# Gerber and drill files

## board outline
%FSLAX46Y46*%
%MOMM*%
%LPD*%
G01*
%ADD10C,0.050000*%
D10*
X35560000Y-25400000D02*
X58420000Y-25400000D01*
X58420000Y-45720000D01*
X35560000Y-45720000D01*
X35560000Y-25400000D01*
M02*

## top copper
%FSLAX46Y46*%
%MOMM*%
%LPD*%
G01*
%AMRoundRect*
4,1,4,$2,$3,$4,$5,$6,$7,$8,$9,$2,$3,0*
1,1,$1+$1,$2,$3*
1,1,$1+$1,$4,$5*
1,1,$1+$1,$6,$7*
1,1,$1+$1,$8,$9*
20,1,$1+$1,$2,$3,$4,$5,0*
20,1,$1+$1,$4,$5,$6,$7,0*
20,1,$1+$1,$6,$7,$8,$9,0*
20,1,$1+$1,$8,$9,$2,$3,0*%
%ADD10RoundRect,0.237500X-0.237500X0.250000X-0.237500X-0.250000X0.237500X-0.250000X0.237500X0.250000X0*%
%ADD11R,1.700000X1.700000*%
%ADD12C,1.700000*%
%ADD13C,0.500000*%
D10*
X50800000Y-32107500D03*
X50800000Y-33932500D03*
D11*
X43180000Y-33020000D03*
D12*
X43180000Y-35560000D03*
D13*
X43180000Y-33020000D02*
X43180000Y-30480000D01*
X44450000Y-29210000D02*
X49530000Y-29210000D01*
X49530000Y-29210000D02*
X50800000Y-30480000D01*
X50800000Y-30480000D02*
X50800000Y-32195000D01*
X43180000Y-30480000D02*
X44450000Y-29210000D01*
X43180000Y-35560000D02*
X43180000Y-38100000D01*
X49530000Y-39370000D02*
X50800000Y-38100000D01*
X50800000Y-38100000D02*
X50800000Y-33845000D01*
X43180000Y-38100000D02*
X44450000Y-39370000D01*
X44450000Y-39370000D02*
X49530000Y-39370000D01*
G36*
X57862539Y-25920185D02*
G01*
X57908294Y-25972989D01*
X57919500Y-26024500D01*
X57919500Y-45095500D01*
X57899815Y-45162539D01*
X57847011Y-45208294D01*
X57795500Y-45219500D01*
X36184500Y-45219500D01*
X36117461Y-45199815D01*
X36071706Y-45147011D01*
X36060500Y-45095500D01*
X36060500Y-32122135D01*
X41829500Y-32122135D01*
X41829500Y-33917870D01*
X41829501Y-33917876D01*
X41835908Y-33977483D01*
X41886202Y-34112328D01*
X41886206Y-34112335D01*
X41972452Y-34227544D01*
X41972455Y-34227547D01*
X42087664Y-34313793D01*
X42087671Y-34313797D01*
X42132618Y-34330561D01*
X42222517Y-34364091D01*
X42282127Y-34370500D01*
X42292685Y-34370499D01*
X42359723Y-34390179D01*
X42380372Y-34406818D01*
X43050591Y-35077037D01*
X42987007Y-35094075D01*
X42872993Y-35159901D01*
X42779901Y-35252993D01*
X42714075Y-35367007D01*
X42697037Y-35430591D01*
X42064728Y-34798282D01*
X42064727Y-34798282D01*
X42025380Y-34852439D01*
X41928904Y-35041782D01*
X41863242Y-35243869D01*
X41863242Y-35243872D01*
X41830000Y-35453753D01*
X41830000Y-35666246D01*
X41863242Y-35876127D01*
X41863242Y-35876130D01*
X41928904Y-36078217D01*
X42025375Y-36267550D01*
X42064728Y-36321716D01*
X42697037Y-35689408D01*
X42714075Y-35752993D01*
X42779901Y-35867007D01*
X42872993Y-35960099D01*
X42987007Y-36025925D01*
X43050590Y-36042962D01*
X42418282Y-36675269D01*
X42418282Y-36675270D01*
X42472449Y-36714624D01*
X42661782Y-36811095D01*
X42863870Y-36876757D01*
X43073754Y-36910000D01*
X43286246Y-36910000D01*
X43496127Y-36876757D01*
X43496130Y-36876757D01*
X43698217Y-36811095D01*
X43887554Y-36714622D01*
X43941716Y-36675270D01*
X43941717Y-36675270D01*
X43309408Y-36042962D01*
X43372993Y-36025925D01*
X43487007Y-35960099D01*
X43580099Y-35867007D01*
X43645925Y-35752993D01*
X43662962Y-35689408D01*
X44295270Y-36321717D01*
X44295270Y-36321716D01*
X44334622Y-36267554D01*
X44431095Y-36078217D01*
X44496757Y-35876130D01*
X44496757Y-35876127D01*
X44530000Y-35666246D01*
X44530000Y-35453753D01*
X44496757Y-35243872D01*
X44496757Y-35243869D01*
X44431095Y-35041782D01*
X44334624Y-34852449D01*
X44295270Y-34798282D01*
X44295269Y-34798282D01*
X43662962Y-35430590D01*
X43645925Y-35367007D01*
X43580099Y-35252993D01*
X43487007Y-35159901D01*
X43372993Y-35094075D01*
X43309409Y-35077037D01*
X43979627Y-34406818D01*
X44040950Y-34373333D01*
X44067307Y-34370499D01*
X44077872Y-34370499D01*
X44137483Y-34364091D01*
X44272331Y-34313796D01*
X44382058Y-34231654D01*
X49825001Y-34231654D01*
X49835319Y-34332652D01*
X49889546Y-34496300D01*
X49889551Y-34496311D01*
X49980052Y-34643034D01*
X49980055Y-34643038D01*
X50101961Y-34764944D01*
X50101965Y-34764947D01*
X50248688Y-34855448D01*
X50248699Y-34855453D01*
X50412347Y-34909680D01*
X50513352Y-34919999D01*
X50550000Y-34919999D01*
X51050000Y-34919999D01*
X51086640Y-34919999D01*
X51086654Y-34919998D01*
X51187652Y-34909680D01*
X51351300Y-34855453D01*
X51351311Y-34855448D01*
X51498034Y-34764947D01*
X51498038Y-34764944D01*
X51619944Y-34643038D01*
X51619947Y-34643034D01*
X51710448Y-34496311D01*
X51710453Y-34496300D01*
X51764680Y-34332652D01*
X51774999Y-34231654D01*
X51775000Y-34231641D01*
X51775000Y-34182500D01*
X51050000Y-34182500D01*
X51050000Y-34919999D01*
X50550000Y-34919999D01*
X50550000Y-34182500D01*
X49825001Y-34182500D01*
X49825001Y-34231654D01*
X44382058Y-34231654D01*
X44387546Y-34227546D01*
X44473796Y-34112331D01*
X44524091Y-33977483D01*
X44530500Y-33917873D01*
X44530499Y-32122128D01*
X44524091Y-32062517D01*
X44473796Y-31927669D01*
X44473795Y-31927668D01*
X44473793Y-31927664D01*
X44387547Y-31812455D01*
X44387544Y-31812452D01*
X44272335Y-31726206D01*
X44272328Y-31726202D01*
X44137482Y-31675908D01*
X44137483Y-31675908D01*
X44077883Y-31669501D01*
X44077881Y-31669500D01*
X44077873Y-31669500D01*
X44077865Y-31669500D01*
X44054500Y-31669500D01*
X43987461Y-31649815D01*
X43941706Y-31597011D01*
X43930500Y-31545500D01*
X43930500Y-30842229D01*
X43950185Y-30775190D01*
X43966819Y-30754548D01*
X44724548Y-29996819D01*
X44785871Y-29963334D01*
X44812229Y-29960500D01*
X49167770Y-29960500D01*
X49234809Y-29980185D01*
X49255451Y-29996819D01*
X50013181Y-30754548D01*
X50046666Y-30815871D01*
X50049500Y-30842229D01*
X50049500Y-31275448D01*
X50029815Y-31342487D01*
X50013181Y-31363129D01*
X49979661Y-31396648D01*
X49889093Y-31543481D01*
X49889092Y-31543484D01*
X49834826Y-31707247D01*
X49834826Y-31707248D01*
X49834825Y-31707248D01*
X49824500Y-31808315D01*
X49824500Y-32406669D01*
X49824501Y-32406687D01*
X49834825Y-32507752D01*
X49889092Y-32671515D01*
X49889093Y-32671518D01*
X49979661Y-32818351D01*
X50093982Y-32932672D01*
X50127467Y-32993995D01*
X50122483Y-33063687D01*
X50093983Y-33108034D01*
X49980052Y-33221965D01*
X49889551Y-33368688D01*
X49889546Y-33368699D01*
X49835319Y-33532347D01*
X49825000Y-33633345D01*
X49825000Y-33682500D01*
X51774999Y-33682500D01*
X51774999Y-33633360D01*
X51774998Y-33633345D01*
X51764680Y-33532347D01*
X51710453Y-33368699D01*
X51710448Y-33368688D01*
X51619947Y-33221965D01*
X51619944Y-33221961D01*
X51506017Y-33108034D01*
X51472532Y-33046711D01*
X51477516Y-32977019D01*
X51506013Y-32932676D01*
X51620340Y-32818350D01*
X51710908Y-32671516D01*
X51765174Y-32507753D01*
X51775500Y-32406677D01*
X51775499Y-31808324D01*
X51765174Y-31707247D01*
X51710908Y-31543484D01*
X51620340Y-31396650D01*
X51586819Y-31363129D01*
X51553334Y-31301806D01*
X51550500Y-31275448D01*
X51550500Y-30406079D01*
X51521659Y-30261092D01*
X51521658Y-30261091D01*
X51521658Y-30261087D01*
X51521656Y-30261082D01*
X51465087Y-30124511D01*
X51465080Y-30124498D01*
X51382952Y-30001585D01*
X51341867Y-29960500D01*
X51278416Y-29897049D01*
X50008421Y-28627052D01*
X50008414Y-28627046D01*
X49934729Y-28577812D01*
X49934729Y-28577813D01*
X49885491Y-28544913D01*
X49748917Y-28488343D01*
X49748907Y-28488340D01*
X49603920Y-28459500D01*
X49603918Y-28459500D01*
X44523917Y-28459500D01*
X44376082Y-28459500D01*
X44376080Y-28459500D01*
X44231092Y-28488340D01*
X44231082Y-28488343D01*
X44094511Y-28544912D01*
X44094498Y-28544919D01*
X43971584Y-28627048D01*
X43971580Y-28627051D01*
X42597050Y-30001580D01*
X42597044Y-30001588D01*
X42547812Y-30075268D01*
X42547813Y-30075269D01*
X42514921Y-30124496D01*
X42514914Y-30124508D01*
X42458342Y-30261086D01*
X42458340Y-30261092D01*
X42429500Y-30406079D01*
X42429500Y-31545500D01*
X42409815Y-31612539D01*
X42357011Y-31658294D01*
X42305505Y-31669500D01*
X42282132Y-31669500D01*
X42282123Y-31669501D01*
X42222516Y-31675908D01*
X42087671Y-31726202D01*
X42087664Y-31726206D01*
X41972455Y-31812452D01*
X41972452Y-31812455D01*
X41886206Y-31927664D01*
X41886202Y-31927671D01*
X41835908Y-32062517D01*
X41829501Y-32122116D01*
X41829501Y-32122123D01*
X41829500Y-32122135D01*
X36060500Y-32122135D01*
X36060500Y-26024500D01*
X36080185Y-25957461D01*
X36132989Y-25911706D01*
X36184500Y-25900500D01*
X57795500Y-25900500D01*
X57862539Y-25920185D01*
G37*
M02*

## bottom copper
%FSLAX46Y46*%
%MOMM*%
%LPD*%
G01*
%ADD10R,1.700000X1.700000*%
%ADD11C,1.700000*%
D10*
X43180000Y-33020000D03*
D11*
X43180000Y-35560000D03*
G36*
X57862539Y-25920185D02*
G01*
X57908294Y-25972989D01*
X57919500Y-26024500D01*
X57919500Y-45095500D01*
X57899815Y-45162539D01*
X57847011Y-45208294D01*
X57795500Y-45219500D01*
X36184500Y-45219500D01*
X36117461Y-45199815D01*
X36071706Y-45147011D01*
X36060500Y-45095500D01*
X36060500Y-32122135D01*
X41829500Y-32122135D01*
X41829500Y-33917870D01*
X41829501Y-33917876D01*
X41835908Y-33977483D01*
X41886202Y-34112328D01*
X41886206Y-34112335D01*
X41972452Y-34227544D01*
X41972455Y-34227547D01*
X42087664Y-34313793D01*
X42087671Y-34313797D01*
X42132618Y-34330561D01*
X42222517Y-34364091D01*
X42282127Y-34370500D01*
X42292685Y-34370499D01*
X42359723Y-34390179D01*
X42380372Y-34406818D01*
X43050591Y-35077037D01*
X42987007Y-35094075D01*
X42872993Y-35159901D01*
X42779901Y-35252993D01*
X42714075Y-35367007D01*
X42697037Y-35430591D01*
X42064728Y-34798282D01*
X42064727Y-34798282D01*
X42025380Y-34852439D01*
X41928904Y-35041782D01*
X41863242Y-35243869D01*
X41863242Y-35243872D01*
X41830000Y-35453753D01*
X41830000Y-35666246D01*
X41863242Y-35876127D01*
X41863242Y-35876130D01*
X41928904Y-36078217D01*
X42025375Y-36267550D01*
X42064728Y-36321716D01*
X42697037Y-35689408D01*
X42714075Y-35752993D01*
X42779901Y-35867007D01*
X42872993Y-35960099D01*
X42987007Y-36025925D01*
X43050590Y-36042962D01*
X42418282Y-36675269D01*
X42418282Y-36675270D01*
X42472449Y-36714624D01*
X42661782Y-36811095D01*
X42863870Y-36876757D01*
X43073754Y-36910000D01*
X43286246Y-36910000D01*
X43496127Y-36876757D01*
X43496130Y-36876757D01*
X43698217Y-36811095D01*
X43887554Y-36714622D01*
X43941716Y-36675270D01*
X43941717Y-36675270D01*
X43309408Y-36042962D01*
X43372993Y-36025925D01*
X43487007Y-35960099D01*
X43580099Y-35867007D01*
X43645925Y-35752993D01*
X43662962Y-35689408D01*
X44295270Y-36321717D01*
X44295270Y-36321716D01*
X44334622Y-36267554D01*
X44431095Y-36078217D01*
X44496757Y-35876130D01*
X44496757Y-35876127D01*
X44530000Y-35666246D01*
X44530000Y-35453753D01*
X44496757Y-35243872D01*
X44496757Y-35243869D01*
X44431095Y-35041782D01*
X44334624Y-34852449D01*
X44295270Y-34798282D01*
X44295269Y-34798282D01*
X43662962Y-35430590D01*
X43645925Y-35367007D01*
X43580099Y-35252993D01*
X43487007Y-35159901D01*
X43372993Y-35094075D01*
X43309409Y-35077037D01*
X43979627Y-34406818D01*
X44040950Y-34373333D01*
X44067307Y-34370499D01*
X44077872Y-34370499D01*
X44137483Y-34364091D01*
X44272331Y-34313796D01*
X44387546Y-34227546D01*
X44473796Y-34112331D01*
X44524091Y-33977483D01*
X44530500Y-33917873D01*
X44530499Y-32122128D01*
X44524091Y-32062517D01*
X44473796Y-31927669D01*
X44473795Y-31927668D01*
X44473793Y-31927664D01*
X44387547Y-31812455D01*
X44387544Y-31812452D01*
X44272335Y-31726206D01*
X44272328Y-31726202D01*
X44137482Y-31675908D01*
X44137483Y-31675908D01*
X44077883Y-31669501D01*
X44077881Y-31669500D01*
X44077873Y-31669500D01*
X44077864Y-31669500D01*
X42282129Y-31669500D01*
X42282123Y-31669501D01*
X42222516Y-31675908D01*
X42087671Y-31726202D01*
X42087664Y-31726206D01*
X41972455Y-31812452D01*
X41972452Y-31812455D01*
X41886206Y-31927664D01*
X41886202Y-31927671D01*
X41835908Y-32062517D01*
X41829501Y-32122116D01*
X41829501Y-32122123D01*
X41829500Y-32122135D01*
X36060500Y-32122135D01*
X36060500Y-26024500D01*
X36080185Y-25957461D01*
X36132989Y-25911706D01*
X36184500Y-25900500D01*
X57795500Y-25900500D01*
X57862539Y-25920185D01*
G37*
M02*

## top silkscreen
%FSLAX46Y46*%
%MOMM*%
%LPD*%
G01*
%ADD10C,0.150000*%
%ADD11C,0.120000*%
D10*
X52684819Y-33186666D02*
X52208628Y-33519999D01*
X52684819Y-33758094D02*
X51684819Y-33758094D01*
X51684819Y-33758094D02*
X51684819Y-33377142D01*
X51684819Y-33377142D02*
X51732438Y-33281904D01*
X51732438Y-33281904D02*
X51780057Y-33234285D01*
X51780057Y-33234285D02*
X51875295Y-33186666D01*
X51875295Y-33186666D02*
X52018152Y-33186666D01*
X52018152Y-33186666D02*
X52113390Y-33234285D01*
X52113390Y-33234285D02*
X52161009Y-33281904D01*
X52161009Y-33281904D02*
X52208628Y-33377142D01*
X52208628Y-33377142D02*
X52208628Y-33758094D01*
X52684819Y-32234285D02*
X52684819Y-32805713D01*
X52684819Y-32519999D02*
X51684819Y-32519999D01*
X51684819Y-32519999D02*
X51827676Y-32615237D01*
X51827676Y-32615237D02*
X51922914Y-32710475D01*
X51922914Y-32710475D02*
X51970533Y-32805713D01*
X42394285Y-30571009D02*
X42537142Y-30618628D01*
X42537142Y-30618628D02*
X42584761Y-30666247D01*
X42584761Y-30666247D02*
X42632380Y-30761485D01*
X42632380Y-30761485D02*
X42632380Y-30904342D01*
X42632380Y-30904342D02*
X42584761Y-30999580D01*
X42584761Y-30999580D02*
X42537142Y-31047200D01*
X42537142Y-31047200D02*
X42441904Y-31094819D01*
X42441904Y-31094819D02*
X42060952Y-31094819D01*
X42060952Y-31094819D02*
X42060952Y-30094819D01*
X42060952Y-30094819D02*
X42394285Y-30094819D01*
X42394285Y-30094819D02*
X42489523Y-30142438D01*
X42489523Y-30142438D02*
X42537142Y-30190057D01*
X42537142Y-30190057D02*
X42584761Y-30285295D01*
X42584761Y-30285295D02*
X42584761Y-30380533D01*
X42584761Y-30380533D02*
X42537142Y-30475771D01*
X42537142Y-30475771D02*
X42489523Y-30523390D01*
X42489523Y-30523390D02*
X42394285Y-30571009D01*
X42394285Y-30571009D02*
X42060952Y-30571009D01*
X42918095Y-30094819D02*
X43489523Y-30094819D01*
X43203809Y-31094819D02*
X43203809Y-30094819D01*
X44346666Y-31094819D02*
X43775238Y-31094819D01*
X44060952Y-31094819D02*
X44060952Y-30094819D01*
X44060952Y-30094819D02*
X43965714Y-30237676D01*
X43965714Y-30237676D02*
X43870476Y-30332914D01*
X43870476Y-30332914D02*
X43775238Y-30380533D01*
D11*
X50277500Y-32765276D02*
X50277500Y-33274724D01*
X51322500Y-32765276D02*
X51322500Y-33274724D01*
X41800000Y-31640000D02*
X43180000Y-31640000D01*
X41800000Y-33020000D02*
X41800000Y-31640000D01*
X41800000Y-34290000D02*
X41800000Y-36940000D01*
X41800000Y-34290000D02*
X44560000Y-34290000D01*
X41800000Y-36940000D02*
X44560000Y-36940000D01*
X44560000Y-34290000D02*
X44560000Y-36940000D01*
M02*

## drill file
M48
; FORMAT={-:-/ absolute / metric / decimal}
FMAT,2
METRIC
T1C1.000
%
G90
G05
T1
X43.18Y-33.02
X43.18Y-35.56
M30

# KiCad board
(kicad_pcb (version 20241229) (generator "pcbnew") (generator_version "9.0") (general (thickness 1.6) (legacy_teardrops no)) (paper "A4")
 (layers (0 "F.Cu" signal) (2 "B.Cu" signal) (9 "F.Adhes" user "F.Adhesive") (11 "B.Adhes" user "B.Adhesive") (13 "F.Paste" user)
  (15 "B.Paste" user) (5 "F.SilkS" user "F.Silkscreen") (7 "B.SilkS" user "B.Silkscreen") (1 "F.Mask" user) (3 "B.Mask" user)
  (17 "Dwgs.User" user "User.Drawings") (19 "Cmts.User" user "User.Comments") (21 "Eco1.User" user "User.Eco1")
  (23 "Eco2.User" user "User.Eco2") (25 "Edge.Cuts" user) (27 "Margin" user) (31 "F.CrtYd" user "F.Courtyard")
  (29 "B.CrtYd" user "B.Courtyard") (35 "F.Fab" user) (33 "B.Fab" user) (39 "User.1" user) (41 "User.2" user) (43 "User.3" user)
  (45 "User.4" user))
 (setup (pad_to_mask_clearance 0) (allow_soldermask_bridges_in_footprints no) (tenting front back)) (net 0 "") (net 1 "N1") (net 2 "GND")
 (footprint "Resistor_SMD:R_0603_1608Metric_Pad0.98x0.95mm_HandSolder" (layer "F.Cu") (at 50.8 33.02 -90)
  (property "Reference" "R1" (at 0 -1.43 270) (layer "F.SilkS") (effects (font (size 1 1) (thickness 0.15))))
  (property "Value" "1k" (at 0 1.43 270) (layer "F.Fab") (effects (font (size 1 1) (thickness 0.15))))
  (fp_line (start -0.254724 0.5225) (end 0.254724 0.5225) (stroke (width 0.12) (type solid)) (layer "F.SilkS"))
  (fp_line (start -0.254724 -0.5225) (end 0.254724 -0.5225) (stroke (width 0.12) (type solid)) (layer "F.SilkS"))
  (pad "1" smd roundrect (at -0.9125 0 270) (size 0.975 0.95) (layers "F.Cu" "F.Mask" "F.Paste") (roundrect_rratio 0.25) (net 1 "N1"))
  (pad "2" smd roundrect (at 0.9125 0 270) (size 0.975 0.95) (layers "F.Cu" "F.Mask" "F.Paste") (roundrect_rratio 0.25) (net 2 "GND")))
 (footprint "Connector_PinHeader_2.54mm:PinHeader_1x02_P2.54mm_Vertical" (layer "F.Cu") (at 43.18 33.02)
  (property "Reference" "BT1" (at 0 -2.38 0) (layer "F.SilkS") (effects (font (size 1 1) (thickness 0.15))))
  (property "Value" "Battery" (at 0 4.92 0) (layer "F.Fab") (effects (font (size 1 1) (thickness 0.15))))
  (fp_line (start -1.38 -1.38) (end 0 -1.38) (stroke (width 0.12) (type solid)) (layer "F.SilkS"))
  (fp_line (start -1.38 0) (end -1.38 -1.38) (stroke (width 0.12) (type solid)) (layer "F.SilkS"))
  (fp_line (start -1.38 1.27) (end -1.38 3.92) (stroke (width 0.12) (type solid)) (layer "F.SilkS"))
  (fp_line (start -1.38 1.27) (end 1.38 1.27) (stroke (width 0.12) (type solid)) (layer "F.SilkS"))
  (fp_line (start -1.38 3.92) (end 1.38 3.92) (stroke (width 0.12) (type solid)) (layer "F.SilkS"))
  (fp_line (start 1.38 1.27) (end 1.38 3.92) (stroke (width 0.12) (type solid)) (layer "F.SilkS"))
  (pad "1" thru_hole rect (at 0 0) (size 1.7 1.7) (drill 1) (layers "*.Cu" "*.Mask") (remove_unused_layers no) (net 1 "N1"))
  (pad "2" thru_hole circle (at 0 2.54) (size 1.7 1.7) (drill 1) (layers "*.Cu" "*.Mask") (remove_unused_layers no) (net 2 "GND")))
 (gr_rect (start 35.56 25.4) (end 58.42 45.72) (stroke (width 0.05) (type default)) (fill no) (layer "Edge.Cuts"))
 (segment (start 43.18 33.02) (end 43.18 30.48) (width 0.5) (layer "F.Cu") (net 1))
 (segment (start 44.45 29.21) (end 49.53 29.21) (width 0.5) (layer "F.Cu") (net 1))
 (segment (start 49.53 29.21) (end 50.8 30.48) (width 0.5) (layer "F.Cu") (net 1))
 (segment (start 50.8 30.48) (end 50.8 32.195) (width 0.5) (layer "F.Cu") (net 1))
 (segment (start 43.18 30.48) (end 44.45 29.21) (width 0.5) (layer "F.Cu") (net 1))
 (segment (start 43.18 35.56) (end 43.18 38.1) (width 0.5) (layer "F.Cu") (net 2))
 (segment (start 49.53 39.37) (end 50.8 38.1) (width 0.5) (layer "F.Cu") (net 2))
 (segment (start 50.8 38.1) (end 50.8 33.845) (width 0.5) (layer "F.Cu") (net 2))
 (segment (start 43.18 38.1) (end 44.45 39.37) (width 0.5) (layer "F.Cu") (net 2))
 (segment (start 44.45 39.37) (end 49.53 39.37) (width 0.5) (layer "F.Cu") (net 2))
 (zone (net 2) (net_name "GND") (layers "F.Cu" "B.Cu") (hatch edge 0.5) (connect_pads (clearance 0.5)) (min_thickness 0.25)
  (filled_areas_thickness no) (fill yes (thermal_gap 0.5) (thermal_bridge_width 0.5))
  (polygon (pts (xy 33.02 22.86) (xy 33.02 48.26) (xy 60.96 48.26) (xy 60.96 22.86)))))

